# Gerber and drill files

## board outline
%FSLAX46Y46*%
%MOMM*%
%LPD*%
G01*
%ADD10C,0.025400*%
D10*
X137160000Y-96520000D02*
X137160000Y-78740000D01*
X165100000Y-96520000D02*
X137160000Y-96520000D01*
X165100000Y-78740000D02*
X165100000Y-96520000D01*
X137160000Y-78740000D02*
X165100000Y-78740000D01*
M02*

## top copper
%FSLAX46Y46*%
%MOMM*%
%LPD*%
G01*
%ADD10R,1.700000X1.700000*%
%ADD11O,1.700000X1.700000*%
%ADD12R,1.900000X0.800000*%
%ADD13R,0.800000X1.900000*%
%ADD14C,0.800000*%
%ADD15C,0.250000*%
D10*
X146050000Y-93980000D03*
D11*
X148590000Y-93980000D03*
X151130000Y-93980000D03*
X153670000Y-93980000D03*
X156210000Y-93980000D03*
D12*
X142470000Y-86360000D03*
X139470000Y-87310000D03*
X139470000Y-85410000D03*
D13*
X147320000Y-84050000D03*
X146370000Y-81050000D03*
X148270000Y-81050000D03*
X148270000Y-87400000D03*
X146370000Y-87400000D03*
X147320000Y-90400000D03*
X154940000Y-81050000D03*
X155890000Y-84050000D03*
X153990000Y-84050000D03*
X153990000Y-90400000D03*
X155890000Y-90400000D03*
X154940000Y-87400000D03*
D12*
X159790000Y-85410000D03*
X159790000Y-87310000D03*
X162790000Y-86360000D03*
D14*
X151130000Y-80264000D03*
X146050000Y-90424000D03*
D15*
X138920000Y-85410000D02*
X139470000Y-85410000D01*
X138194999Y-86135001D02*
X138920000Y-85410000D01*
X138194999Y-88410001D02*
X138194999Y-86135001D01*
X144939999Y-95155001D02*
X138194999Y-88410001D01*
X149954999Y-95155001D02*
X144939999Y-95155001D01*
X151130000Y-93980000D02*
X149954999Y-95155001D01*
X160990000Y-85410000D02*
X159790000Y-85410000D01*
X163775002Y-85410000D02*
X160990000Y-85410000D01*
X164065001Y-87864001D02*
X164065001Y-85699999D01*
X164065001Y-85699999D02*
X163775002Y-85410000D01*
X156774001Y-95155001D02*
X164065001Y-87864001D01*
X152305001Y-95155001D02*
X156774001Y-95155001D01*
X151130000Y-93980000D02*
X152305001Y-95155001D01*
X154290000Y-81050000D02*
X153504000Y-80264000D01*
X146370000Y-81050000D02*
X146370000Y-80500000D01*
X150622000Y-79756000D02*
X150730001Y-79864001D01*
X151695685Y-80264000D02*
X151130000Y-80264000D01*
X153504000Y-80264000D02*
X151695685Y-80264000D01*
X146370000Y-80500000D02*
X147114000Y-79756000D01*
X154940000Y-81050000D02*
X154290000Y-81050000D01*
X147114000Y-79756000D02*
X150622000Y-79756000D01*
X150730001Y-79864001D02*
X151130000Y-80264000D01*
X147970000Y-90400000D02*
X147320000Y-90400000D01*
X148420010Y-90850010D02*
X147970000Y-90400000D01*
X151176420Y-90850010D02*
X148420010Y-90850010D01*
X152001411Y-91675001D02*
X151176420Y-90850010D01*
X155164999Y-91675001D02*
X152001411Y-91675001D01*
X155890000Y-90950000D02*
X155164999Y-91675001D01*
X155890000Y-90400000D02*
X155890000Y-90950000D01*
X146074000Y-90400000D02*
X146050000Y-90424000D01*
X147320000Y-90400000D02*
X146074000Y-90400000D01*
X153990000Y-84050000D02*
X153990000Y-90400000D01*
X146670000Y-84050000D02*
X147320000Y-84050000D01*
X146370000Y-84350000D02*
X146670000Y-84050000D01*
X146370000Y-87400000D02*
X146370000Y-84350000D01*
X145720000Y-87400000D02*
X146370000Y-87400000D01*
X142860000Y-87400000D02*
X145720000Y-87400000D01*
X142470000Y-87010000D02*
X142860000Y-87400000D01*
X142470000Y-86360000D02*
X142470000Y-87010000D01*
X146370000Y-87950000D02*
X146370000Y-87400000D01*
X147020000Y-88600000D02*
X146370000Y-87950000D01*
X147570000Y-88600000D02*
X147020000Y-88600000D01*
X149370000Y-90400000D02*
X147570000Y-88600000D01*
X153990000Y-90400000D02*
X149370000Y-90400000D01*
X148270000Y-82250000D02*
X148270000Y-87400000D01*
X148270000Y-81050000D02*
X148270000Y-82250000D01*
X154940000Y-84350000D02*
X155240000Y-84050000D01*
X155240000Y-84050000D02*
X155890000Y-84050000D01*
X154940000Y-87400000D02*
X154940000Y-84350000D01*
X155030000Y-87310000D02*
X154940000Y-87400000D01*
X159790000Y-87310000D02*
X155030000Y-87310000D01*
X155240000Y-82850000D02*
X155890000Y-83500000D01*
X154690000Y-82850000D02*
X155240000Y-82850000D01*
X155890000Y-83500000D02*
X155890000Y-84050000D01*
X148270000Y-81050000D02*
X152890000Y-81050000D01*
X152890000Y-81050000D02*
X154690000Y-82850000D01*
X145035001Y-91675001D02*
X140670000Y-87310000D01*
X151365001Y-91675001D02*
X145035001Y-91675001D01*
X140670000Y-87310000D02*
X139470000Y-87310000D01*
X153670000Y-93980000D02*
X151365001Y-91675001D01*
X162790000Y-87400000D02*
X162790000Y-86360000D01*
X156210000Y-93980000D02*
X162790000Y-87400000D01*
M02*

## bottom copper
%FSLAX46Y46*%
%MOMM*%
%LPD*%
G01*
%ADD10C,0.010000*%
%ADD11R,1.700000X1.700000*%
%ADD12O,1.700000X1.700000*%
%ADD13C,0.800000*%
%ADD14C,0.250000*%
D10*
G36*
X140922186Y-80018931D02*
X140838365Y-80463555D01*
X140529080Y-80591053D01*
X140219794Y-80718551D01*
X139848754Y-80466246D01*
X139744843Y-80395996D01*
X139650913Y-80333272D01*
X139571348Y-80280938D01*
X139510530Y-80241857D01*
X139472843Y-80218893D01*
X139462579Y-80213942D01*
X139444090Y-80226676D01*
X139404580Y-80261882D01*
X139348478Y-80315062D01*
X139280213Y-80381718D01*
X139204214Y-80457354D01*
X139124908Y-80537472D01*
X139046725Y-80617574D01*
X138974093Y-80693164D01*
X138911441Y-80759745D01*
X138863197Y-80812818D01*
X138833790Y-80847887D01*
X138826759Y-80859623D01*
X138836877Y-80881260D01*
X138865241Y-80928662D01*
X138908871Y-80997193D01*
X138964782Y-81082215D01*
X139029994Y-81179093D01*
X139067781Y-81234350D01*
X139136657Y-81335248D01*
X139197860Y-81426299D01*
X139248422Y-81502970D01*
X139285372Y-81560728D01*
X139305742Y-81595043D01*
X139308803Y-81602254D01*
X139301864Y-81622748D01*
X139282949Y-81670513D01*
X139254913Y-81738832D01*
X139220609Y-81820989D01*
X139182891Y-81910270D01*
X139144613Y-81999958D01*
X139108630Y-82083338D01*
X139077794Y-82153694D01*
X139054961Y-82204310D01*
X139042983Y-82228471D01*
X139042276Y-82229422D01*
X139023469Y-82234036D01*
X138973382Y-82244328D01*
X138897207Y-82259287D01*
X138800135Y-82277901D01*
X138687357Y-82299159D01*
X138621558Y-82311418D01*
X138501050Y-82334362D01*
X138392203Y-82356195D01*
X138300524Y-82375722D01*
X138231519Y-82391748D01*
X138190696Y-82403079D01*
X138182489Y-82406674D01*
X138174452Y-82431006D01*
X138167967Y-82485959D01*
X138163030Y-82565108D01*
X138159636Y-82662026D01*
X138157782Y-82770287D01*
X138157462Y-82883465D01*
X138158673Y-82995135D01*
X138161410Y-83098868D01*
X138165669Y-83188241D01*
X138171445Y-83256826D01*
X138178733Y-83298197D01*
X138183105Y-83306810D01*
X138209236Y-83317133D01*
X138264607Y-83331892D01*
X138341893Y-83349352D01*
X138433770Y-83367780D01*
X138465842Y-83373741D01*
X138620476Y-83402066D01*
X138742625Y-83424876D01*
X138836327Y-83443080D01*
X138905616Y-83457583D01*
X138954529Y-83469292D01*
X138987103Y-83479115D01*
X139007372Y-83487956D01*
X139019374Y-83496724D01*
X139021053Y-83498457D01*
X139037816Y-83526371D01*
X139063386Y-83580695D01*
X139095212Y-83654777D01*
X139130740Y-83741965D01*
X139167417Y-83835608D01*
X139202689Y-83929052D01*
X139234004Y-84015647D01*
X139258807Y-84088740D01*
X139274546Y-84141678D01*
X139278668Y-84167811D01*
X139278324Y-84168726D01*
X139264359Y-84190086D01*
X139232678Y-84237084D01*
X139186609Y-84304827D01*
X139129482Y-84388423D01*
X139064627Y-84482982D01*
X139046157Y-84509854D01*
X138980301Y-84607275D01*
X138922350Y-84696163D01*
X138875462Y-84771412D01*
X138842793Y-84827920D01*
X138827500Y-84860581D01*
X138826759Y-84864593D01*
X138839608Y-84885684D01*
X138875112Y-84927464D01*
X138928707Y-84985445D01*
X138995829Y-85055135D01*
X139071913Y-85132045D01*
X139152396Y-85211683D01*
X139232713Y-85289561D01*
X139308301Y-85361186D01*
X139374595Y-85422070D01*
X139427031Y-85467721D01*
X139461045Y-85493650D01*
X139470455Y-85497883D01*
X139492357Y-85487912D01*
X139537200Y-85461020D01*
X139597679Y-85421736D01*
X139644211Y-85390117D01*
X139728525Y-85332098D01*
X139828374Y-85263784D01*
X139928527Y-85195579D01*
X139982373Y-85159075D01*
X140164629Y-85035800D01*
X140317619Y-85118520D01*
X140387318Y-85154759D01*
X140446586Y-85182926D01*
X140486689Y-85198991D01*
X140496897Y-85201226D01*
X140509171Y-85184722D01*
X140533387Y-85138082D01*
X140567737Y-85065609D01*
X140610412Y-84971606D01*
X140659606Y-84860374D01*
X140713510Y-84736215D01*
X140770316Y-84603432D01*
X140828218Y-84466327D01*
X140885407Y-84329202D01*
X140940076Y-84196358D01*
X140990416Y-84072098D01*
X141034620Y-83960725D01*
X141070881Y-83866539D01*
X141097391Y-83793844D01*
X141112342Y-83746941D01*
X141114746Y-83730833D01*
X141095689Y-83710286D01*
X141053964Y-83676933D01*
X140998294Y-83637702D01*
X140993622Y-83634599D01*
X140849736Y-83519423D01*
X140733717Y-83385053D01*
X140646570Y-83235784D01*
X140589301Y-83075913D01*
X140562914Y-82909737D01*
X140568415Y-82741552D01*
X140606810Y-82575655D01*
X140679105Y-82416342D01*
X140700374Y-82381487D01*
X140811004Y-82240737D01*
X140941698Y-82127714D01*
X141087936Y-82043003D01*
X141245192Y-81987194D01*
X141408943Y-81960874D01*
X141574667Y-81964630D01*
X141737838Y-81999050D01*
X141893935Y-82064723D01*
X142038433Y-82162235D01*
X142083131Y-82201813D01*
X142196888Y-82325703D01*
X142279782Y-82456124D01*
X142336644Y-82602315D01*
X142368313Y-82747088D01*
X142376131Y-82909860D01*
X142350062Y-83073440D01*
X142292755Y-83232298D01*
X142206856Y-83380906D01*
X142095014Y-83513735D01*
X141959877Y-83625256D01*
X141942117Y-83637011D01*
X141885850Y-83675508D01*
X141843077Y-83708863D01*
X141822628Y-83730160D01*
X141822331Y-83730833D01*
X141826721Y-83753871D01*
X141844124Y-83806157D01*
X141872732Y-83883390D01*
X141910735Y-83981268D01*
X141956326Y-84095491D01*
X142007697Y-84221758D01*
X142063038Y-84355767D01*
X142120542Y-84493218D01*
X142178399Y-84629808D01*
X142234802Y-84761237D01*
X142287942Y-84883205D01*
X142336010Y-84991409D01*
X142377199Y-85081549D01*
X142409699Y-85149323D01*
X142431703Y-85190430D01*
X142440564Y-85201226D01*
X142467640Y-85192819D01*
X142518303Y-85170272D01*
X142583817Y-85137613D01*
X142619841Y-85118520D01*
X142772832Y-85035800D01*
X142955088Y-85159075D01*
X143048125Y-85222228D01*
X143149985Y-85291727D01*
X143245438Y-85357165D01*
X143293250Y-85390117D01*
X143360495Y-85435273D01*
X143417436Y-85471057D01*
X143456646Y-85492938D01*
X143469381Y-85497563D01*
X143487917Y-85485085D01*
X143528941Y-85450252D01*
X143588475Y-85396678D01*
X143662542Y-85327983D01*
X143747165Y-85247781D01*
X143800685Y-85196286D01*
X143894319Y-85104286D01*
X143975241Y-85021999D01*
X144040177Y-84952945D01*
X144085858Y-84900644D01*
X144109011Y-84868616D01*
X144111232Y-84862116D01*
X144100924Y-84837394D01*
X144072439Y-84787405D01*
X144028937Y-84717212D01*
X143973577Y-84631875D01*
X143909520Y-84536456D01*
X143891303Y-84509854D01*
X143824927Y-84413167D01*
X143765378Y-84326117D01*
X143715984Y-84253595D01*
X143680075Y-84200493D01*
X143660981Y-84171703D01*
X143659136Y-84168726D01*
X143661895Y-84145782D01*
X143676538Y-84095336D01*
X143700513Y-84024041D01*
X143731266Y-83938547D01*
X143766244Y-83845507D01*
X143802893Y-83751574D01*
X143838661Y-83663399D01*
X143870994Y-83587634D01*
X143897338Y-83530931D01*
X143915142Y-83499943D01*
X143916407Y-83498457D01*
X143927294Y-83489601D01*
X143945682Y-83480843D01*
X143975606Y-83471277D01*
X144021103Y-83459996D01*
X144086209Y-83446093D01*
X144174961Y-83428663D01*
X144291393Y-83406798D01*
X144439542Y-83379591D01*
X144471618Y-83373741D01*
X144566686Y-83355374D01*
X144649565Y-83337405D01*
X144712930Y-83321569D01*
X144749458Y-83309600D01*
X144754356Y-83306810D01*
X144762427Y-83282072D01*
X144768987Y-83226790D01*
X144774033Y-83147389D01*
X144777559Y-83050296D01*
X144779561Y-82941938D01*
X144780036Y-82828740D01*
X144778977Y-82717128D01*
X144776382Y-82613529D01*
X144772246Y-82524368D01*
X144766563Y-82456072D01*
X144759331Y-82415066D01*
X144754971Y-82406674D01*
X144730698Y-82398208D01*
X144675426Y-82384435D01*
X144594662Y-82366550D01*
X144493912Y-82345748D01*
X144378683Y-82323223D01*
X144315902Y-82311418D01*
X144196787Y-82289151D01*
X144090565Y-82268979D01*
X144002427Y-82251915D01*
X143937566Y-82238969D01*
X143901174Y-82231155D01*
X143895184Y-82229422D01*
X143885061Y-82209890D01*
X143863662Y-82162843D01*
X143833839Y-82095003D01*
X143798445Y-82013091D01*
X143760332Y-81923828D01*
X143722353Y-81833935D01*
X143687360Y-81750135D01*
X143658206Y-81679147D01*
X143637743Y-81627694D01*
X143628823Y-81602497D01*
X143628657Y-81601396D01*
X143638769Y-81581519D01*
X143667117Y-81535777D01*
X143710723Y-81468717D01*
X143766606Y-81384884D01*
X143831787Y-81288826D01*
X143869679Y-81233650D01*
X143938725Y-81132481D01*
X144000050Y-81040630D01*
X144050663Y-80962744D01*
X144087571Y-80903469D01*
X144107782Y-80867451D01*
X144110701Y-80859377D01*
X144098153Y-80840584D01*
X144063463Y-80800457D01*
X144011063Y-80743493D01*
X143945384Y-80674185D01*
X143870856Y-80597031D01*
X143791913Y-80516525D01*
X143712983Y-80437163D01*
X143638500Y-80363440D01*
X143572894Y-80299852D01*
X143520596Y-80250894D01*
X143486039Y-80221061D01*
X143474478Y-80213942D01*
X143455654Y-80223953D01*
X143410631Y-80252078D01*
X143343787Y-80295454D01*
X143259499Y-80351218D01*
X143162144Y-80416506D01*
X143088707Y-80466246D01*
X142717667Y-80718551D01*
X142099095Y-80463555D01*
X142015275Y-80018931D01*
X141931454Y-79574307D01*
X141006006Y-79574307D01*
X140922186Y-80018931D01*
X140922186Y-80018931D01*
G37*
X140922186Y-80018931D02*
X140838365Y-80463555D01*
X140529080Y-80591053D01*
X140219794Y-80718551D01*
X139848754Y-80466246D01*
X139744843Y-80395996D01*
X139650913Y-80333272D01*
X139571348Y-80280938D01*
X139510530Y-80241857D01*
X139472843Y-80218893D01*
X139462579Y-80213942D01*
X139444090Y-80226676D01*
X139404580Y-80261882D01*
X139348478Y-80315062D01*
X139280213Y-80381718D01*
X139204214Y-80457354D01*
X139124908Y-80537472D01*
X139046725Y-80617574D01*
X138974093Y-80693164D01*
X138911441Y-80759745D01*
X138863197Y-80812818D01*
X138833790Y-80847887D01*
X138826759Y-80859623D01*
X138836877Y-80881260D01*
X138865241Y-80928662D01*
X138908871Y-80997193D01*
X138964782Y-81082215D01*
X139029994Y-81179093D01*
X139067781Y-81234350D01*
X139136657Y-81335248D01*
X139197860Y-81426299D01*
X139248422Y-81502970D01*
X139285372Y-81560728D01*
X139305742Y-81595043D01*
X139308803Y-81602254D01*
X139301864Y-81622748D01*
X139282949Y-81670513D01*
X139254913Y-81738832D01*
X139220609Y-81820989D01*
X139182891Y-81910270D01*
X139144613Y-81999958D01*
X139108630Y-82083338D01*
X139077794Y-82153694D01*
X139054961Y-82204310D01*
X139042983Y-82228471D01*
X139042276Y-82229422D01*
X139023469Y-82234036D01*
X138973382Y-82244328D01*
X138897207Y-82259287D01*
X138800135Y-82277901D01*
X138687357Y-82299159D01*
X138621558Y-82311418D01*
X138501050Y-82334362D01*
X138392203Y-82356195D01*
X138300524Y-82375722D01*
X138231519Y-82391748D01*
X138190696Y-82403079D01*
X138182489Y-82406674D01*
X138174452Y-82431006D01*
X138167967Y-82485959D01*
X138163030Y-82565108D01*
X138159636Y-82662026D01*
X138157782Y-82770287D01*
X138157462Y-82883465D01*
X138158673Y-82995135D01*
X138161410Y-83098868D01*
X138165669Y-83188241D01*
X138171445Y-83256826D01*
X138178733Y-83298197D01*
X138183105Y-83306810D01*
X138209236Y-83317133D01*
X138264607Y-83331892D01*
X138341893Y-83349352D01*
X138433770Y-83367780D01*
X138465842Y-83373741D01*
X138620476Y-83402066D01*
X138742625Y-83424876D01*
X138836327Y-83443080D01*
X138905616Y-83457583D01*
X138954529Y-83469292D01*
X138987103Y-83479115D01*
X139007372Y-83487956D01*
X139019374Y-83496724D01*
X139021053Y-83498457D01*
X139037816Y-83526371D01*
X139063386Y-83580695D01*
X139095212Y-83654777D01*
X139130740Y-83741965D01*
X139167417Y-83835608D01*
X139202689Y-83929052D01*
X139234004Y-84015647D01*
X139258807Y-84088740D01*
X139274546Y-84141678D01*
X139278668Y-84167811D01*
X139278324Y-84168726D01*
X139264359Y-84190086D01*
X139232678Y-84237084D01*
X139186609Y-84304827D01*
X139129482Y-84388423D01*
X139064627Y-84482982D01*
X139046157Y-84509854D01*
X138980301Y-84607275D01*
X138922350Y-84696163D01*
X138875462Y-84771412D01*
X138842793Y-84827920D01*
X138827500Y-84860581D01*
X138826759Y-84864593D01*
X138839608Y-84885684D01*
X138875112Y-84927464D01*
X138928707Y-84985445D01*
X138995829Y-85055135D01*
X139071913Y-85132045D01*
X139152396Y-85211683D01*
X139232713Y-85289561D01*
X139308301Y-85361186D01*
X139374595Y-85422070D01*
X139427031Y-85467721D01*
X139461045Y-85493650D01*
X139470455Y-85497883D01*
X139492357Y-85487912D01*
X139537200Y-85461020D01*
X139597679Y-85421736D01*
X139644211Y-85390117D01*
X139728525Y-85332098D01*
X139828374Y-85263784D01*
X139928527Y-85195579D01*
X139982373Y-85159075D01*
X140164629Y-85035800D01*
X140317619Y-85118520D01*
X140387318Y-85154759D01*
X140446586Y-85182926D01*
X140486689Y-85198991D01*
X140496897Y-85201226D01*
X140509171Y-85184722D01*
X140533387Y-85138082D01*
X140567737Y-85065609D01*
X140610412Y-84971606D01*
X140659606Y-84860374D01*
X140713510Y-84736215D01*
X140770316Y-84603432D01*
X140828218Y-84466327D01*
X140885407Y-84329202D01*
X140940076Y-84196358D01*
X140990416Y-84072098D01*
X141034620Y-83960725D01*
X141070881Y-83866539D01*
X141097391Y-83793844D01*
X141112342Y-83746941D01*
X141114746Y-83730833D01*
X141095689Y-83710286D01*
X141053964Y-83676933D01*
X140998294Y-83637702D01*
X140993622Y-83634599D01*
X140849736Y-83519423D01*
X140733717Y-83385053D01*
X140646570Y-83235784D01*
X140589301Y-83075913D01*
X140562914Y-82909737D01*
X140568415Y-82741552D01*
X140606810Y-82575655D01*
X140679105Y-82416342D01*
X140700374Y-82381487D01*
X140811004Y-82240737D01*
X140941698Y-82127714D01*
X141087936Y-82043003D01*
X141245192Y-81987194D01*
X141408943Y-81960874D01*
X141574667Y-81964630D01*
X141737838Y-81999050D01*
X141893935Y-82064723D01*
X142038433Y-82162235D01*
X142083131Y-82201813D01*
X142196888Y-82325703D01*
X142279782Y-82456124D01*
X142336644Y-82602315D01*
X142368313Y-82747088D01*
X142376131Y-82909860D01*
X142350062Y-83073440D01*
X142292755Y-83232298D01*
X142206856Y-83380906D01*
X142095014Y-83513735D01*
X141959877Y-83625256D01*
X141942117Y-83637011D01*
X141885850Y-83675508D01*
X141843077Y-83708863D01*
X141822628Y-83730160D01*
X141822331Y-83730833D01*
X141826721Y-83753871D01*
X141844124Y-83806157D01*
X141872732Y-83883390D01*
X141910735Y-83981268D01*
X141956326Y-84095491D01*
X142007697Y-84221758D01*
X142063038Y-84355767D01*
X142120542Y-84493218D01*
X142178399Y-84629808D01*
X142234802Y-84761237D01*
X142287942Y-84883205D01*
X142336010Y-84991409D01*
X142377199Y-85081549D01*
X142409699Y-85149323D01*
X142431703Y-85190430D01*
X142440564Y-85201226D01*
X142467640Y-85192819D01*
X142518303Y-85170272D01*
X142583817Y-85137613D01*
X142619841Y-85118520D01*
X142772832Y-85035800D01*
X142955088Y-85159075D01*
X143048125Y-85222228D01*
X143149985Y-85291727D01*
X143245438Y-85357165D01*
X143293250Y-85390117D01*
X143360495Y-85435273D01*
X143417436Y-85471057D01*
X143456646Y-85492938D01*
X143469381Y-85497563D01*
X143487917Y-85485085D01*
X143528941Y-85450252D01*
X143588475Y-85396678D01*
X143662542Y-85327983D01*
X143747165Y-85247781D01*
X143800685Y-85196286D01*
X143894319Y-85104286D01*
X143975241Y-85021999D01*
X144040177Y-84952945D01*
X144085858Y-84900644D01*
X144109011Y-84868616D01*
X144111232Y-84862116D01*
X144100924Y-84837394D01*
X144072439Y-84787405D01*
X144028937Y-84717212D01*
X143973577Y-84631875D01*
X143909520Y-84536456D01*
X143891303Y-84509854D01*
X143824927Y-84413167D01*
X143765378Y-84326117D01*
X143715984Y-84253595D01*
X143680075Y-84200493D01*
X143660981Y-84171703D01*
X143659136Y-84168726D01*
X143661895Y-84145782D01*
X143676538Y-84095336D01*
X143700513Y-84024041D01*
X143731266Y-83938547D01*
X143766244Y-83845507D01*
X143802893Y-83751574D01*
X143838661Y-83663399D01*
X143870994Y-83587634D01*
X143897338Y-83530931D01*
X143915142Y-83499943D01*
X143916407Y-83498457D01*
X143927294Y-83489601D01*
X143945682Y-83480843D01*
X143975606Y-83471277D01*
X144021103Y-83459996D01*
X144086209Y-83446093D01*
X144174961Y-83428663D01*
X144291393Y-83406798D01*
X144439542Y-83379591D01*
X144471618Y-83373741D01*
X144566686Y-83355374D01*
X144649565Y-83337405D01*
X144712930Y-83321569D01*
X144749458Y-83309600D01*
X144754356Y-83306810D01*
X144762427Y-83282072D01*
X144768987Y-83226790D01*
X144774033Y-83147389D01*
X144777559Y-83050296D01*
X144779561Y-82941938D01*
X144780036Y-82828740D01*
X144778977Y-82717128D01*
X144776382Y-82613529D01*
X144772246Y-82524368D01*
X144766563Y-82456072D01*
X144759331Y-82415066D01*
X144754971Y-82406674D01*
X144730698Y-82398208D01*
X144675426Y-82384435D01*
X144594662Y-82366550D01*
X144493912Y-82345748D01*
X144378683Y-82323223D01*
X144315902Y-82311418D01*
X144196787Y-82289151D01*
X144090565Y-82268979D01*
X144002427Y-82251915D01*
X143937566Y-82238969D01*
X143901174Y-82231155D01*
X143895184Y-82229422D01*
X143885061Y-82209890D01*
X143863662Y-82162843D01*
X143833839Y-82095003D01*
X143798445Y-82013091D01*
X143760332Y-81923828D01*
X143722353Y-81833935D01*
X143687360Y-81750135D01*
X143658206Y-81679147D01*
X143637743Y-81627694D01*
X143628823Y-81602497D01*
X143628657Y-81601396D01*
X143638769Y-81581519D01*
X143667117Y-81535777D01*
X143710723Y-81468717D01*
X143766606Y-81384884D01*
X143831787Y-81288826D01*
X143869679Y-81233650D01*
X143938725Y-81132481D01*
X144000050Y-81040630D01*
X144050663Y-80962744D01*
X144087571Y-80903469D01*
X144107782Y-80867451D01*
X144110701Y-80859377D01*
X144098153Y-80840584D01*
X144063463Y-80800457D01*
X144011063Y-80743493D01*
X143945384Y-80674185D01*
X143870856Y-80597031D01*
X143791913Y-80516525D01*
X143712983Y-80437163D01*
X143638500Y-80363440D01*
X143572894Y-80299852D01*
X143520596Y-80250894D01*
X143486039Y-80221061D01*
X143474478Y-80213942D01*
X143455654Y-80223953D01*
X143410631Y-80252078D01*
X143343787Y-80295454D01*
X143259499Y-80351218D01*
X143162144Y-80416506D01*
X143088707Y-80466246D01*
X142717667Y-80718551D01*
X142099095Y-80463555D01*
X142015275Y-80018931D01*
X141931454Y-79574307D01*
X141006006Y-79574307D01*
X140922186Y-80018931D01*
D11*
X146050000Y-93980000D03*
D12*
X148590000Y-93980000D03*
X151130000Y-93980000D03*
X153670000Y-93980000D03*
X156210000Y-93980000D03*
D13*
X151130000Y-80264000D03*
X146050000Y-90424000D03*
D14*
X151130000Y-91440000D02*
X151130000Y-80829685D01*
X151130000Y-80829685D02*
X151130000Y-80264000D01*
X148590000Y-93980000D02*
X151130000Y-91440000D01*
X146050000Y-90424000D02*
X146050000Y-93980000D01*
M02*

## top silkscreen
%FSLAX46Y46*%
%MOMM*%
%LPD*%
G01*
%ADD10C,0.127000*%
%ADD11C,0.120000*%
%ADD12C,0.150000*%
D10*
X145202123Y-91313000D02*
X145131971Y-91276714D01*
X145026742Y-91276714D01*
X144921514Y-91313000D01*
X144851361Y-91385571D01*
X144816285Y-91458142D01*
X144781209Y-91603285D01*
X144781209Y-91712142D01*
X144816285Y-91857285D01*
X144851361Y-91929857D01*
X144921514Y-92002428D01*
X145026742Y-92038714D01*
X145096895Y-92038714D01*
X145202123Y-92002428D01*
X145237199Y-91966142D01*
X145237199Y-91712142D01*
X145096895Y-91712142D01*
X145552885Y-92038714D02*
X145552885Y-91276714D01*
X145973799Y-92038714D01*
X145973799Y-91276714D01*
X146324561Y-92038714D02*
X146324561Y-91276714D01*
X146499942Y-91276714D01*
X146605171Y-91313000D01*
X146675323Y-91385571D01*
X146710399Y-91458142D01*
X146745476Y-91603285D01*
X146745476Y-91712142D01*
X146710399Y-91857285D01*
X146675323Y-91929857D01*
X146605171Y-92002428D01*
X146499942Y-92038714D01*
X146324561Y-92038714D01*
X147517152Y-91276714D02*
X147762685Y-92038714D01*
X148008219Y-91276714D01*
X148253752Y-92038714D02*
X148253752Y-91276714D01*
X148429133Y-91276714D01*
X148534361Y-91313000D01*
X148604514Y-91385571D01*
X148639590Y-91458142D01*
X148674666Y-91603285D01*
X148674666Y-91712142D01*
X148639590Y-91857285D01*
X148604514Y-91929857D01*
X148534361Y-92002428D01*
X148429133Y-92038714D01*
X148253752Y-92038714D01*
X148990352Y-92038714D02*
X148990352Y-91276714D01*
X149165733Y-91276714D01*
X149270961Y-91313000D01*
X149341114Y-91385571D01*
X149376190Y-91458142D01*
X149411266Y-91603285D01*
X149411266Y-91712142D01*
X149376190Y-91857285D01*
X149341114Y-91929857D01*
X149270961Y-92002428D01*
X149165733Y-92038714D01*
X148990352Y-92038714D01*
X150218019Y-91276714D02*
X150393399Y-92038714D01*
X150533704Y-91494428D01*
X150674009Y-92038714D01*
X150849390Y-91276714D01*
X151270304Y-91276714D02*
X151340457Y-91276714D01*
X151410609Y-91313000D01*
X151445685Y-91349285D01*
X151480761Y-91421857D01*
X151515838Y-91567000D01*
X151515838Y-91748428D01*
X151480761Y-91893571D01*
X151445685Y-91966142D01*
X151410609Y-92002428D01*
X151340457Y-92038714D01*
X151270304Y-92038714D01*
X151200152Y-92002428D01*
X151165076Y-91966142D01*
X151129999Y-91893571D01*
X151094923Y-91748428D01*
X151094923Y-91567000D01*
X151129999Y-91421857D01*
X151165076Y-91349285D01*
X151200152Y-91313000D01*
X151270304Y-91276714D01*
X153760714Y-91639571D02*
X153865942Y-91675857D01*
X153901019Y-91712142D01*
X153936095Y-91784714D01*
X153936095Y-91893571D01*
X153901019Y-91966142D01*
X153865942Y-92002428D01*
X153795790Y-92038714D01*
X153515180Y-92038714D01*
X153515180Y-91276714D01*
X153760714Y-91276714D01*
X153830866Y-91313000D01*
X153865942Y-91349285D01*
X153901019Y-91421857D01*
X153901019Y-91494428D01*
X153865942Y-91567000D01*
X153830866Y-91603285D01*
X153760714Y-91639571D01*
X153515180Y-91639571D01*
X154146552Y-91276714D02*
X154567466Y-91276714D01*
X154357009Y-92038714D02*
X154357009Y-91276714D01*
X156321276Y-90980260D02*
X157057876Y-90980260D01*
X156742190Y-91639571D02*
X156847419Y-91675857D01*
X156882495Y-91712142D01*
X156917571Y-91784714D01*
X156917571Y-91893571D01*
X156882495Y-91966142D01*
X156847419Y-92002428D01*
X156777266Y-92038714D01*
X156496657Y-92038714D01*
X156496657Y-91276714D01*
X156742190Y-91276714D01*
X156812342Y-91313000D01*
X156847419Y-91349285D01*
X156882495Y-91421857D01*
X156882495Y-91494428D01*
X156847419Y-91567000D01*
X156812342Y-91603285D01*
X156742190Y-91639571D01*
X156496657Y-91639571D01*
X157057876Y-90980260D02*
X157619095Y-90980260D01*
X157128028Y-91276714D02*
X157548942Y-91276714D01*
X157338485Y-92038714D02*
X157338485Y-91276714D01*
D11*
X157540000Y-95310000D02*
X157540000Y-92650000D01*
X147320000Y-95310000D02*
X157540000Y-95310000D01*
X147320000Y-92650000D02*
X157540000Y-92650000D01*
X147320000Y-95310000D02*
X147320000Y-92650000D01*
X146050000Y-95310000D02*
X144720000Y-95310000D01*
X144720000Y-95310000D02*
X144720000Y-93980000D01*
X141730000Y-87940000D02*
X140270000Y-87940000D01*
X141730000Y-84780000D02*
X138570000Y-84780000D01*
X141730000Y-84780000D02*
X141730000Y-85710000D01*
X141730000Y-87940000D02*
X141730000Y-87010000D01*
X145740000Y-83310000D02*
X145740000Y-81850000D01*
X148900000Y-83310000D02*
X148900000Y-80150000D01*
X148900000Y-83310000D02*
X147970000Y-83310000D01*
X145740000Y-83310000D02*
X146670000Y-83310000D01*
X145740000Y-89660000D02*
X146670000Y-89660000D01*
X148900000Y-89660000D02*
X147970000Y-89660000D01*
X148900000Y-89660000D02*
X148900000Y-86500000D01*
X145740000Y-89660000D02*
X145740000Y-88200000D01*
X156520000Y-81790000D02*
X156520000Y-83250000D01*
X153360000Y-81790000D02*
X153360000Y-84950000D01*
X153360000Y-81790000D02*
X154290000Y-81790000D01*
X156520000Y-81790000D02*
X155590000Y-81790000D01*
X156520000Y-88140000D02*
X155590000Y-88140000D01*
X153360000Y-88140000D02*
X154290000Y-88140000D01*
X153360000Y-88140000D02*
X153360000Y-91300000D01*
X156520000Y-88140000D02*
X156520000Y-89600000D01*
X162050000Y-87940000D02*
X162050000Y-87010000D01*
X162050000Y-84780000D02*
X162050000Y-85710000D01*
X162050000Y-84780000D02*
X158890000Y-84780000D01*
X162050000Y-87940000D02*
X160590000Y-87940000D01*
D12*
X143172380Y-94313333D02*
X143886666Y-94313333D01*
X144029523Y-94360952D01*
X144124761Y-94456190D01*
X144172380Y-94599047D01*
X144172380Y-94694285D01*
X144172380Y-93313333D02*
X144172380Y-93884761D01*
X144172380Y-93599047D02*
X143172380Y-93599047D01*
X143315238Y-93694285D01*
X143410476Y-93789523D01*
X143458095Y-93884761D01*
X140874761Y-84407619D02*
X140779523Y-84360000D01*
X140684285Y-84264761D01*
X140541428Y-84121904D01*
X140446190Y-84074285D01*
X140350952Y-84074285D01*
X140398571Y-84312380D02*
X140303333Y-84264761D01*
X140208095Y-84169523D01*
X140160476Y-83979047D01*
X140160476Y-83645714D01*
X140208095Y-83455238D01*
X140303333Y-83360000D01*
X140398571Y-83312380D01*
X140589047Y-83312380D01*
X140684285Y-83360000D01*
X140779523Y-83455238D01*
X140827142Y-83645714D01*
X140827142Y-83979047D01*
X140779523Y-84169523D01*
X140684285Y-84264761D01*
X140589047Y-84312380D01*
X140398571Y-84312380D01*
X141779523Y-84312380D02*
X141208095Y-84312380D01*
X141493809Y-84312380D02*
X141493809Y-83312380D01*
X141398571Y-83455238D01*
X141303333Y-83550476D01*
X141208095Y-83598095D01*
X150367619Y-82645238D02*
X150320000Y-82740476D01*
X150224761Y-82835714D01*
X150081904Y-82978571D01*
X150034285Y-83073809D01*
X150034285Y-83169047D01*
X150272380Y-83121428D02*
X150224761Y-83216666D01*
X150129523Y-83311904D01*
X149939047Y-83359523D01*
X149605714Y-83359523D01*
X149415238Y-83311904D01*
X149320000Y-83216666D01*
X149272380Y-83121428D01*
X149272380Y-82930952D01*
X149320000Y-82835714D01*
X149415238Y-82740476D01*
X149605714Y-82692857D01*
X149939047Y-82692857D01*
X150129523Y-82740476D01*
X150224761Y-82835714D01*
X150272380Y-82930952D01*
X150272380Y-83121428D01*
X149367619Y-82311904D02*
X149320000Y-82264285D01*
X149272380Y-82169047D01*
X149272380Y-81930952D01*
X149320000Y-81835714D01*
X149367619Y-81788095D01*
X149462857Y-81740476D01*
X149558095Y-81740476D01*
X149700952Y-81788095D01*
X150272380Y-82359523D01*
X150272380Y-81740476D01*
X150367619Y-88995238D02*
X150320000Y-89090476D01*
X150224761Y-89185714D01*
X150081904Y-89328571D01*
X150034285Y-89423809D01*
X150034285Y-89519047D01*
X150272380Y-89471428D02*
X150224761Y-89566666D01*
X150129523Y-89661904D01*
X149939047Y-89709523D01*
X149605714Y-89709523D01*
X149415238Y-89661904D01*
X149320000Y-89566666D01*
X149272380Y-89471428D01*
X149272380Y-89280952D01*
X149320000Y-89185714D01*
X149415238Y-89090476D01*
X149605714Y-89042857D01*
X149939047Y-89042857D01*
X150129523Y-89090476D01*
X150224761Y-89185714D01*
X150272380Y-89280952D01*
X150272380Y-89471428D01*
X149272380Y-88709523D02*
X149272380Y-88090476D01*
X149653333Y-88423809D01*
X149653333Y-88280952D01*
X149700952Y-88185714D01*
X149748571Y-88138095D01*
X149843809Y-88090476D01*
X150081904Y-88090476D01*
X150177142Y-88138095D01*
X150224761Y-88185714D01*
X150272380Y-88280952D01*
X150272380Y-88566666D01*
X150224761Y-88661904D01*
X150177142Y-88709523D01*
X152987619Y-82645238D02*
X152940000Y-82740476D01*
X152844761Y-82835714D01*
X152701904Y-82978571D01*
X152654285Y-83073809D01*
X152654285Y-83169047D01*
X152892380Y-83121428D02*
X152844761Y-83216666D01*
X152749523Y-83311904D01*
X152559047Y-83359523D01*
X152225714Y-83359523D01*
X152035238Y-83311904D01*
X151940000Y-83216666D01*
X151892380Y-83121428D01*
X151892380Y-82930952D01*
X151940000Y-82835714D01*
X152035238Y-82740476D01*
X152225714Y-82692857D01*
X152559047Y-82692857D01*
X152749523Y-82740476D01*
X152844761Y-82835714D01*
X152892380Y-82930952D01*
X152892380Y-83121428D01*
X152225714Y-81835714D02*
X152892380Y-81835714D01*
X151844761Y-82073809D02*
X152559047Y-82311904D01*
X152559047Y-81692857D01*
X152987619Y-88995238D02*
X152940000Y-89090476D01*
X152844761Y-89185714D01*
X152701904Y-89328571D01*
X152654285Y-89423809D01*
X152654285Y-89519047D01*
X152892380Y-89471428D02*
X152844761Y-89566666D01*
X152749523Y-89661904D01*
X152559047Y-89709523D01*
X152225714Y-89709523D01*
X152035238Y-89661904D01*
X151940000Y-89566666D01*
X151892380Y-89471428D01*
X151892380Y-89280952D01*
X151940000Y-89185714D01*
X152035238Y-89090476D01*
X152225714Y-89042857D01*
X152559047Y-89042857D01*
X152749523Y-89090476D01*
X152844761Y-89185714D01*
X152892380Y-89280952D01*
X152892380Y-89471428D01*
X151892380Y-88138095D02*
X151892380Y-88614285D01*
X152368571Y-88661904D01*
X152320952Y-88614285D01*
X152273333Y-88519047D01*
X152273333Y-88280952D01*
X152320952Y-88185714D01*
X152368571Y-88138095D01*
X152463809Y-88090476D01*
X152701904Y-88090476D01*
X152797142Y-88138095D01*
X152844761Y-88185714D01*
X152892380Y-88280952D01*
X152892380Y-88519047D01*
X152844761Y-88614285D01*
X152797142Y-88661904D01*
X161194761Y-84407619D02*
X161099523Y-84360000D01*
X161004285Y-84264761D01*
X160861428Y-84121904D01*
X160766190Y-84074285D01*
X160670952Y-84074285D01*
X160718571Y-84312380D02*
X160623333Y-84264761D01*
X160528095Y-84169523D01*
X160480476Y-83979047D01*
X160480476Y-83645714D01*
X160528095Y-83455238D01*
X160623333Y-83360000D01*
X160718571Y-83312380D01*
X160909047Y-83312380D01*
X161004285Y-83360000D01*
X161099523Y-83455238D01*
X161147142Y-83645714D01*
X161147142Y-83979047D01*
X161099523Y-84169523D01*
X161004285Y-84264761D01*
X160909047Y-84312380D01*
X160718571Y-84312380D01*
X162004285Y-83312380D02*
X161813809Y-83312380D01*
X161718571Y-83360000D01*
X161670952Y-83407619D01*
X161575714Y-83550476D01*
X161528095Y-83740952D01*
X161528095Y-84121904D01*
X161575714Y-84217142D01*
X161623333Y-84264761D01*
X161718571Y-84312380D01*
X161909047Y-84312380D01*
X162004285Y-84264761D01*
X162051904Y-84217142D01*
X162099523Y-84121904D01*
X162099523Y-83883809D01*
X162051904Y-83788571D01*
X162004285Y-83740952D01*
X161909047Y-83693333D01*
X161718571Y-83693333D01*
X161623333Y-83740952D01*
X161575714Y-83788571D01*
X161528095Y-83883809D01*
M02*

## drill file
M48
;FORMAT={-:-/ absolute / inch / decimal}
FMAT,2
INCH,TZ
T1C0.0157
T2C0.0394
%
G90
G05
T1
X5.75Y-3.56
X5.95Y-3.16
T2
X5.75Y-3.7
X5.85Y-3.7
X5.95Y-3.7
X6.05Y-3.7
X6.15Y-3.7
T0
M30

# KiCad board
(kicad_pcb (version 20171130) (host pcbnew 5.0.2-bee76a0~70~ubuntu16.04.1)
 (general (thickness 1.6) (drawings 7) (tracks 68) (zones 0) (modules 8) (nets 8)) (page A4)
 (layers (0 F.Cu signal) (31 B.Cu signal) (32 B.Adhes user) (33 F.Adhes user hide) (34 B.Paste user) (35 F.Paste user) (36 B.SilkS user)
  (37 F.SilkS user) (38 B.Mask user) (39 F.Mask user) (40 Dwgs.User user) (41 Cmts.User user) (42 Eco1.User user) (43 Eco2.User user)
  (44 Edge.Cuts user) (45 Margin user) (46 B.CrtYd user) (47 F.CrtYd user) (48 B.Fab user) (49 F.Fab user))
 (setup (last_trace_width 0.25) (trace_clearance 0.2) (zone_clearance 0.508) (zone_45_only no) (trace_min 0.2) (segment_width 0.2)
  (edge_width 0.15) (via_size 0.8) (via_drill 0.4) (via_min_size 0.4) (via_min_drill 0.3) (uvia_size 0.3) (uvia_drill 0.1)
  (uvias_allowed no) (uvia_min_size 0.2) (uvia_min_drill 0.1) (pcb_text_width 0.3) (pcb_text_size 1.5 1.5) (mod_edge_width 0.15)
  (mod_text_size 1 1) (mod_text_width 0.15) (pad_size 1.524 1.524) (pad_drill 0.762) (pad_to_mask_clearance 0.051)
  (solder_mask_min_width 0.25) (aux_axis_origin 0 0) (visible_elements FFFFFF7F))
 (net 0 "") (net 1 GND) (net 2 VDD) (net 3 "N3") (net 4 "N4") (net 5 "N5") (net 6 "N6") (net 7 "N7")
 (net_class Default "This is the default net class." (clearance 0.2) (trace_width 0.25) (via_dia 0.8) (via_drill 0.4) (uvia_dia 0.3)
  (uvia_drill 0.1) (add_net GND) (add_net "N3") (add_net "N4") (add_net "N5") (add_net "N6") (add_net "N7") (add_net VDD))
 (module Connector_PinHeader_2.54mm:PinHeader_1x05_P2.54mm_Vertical (layer F.Cu) (at 146.05 93.98 90)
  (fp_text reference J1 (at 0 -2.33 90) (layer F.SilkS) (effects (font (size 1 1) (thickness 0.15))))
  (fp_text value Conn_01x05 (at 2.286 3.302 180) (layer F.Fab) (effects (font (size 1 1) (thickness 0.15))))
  (fp_line (start -1.33 11.49) (end 1.33 11.49) (layer F.SilkS) (width 0.12))
  (fp_line (start -1.33 1.27) (end -1.33 11.49) (layer F.SilkS) (width 0.12))
  (fp_line (start 1.33 1.27) (end 1.33 11.49) (layer F.SilkS) (width 0.12))
  (fp_line (start -1.33 1.27) (end 1.33 1.27) (layer F.SilkS) (width 0.12))
  (fp_line (start -1.33 0) (end -1.33 -1.33) (layer F.SilkS) (width 0.12))
  (fp_line (start -1.33 -1.33) (end 0 -1.33) (layer F.SilkS) (width 0.12))
  (pad 1 thru_hole rect (at 0 0 90) (size 1.7 1.7) (drill 1) (layers *.Cu *.Mask) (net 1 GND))
  (pad 2 thru_hole oval (at 0 2.54 90) (size 1.7 1.7) (drill 1) (layers *.Cu *.Mask) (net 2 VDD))
  (pad 3 thru_hole oval (at 0 5.08 90) (size 1.7 1.7) (drill 1) (layers *.Cu *.Mask) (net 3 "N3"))
  (pad 4 thru_hole oval (at 0 7.62 90) (size 1.7 1.7) (drill 1) (layers *.Cu *.Mask) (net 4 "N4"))
  (pad 5 thru_hole oval (at 0 10.16 90) (size 1.7 1.7) (drill 1) (layers *.Cu *.Mask) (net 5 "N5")))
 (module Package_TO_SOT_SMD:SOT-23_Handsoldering (layer F.Cu) (at 140.97 86.36)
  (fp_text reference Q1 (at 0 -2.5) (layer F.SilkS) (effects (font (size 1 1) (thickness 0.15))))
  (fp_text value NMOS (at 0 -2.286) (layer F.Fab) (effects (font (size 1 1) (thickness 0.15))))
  (fp_line (start 0.76 1.58) (end -0.7 1.58) (layer F.SilkS) (width 0.12))
  (fp_line (start 0.76 -1.58) (end -2.4 -1.58) (layer F.SilkS) (width 0.12))
  (fp_line (start 0.76 -1.58) (end 0.76 -0.65) (layer F.SilkS) (width 0.12))
  (fp_line (start 0.76 1.58) (end 0.76 0.65) (layer F.SilkS) (width 0.12))
  (pad 3 smd rect (at 1.5 0) (size 1.9 0.8) (layers F.Cu F.Paste F.Mask) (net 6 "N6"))
  (pad 2 smd rect (at -1.5 0.95) (size 1.9 0.8) (layers F.Cu F.Paste F.Mask) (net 4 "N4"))
  (pad 1 smd rect (at -1.5 -0.95) (size 1.9 0.8) (layers F.Cu F.Paste F.Mask) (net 3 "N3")))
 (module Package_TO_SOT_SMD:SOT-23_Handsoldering (layer F.Cu) (at 147.32 82.55 270)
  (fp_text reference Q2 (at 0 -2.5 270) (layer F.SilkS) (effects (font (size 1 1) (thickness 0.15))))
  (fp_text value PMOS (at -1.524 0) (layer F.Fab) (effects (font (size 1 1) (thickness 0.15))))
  (fp_line (start 0.76 1.58) (end -0.7 1.58) (layer F.SilkS) (width 0.12))
  (fp_line (start 0.76 -1.58) (end -2.4 -1.58) (layer F.SilkS) (width 0.12))
  (fp_line (start 0.76 -1.58) (end 0.76 -0.65) (layer F.SilkS) (width 0.12))
  (fp_line (start 0.76 1.58) (end 0.76 0.65) (layer F.SilkS) (width 0.12))
  (pad 3 smd rect (at 1.5 0 270) (size 1.9 0.8) (layers F.Cu F.Paste F.Mask) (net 6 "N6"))
  (pad 2 smd rect (at -1.5 0.95 270) (size 1.9 0.8) (layers F.Cu F.Paste F.Mask) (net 2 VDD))
  (pad 1 smd rect (at -1.5 -0.95 270) (size 1.9 0.8) (layers F.Cu F.Paste F.Mask) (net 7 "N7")))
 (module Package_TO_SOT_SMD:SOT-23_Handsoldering (layer F.Cu) (at 147.32 88.9 270)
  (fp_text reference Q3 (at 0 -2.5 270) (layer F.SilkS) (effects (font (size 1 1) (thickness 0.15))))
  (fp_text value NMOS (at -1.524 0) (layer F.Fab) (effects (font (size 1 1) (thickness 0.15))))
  (fp_line (start 0.76 1.58) (end 0.76 0.65) (layer F.SilkS) (width 0.12))
  (fp_line (start 0.76 -1.58) (end 0.76 -0.65) (layer F.SilkS) (width 0.12))
  (fp_line (start 0.76 -1.58) (end -2.4 -1.58) (layer F.SilkS) (width 0.12))
  (fp_line (start 0.76 1.58) (end -0.7 1.58) (layer F.SilkS) (width 0.12))
  (pad 1 smd rect (at -1.5 -0.95 270) (size 1.9 0.8) (layers F.Cu F.Paste F.Mask) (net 7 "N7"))
  (pad 2 smd rect (at -1.5 0.95 270) (size 1.9 0.8) (layers F.Cu F.Paste F.Mask) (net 6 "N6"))
  (pad 3 smd rect (at 1.5 0 270) (size 1.9 0.8) (layers F.Cu F.Paste F.Mask) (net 1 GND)))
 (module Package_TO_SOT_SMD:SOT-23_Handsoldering (layer F.Cu) (at 154.94 82.55 90)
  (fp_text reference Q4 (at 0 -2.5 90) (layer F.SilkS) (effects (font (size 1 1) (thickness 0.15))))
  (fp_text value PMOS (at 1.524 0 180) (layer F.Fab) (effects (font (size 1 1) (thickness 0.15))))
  (fp_line (start 0.76 1.58) (end -0.7 1.58) (layer F.SilkS) (width 0.12))
  (fp_line (start 0.76 -1.58) (end -2.4 -1.58) (layer F.SilkS) (width 0.12))
  (fp_line (start 0.76 -1.58) (end 0.76 -0.65) (layer F.SilkS) (width 0.12))
  (fp_line (start 0.76 1.58) (end 0.76 0.65) (layer F.SilkS) (width 0.12))
  (pad 3 smd rect (at 1.5 0 90) (size 1.9 0.8) (layers F.Cu F.Paste F.Mask) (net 2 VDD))
  (pad 2 smd rect (at -1.5 0.95 90) (size 1.9 0.8) (layers F.Cu F.Paste F.Mask) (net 7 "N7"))
  (pad 1 smd rect (at -1.5 -0.95 90) (size 1.9 0.8) (layers F.Cu F.Paste F.Mask) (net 6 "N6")))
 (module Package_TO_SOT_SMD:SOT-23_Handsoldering (layer F.Cu) (at 154.94 88.9 90)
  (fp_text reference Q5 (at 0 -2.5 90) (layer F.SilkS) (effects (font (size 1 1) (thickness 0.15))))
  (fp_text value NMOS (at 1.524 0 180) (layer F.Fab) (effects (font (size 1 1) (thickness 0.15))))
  (fp_line (start 0.76 1.58) (end 0.76 0.65) (layer F.SilkS) (width 0.12))
  (fp_line (start 0.76 -1.58) (end 0.76 -0.65) (layer F.SilkS) (width 0.12))
  (fp_line (start 0.76 -1.58) (end -2.4 -1.58) (layer F.SilkS) (width 0.12))
  (fp_line (start 0.76 1.58) (end -0.7 1.58) (layer F.SilkS) (width 0.12))
  (pad 1 smd rect (at -1.5 -0.95 90) (size 1.9 0.8) (layers F.Cu F.Paste F.Mask) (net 6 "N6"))
  (pad 2 smd rect (at -1.5 0.95 90) (size 1.9 0.8) (layers F.Cu F.Paste F.Mask) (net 1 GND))
  (pad 3 smd rect (at 1.5 0 90) (size 1.9 0.8) (layers F.Cu F.Paste F.Mask) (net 7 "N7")))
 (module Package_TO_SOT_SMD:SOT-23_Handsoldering (layer F.Cu) (at 161.29 86.36)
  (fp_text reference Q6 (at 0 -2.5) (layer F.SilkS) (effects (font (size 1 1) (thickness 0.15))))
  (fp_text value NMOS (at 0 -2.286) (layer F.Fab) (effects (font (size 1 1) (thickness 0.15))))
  (fp_line (start 0.76 1.58) (end 0.76 0.65) (layer F.SilkS) (width 0.12))
  (fp_line (start 0.76 -1.58) (end 0.76 -0.65) (layer F.SilkS) (width 0.12))
  (fp_line (start 0.76 -1.58) (end -2.4 -1.58) (layer F.SilkS) (width 0.12))
  (fp_line (start 0.76 1.58) (end -0.7 1.58) (layer F.SilkS) (width 0.12))
  (pad 1 smd rect (at -1.5 -0.95) (size 1.9 0.8) (layers F.Cu F.Paste F.Mask) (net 3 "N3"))
  (pad 2 smd rect (at -1.5 0.95) (size 1.9 0.8) (layers F.Cu F.Paste F.Mask) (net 7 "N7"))
  (pad 3 smd rect (at 1.5 0) (size 1.9 0.8) (layers F.Cu F.Paste F.Mask) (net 5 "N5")))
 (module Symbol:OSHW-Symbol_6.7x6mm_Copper (layer B.Cu) (at 141.478 82.55 180)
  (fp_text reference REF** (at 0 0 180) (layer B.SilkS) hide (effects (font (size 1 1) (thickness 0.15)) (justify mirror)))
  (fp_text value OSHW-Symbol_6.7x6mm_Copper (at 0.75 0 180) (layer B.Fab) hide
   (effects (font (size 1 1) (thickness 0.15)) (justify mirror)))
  (fp_poly
   (pts (xy 0.555814 2.531069) (xy 0.639635 2.086445) (xy 0.94892 1.958947) (xy 1.258206 1.831449) (xy 1.629246 2.083754)
    (xy 1.733157 2.154004) (xy 1.827087 2.216728) (xy 1.906652 2.269062) (xy 1.96747 2.308143) (xy 2.005157 2.331107) (xy 2.015421 2.336058)
    (xy 2.03391 2.323324) (xy 2.07342 2.288118) (xy 2.129522 2.234938) (xy 2.197787 2.168282) (xy 2.273786 2.092646) (xy 2.353092 2.012528)
    (xy 2.431275 1.932426) (xy 2.503907 1.856836) (xy 2.566559 1.790255) (xy 2.614803 1.737182) (xy 2.64421 1.702113) (xy 2.651241 1.690377)
    (xy 2.641123 1.66874) (xy 2.612759 1.621338) (xy 2.569129 1.552807) (xy 2.513218 1.467785) (xy 2.448006 1.370907) (xy 2.410219 1.31565)
    (xy 2.341343 1.214752) (xy 2.28014 1.123701) (xy 2.229578 1.04703) (xy 2.192628 0.989272) (xy 2.172258 0.954957) (xy 2.169197 0.947746)
    (xy 2.176136 0.927252) (xy 2.195051 0.879487) (xy 2.223087 0.811168) (xy 2.257391 0.729011) (xy 2.295109 0.63973) (xy 2.333387 0.550042)
    (xy 2.36937 0.466662) (xy 2.400206 0.396306) (xy 2.423039 0.34569) (xy 2.435017 0.321529) (xy 2.435724 0.320578) (xy 2.454531 0.315964)
    (xy 2.504618 0.305672) (xy 2.580793 0.290713) (xy 2.677865 0.272099) (xy 2.790643 0.250841) (xy 2.856442 0.238582) (xy 2.97695 0.215638)
    (xy 3.085797 0.193805) (xy 3.177476 0.174278) (xy 3.246481 0.158252) (xy 3.287304 0.146921) (xy 3.295511 0.143326)
    (xy 3.303548 0.118994) (xy 3.310033 0.064041) (xy 3.31497 -0.015108) (xy 3.318364 -0.112026) (xy 3.320218 -0.220287)
    (xy 3.320538 -0.333465) (xy 3.319327 -0.445135) (xy 3.31659 -0.548868) (xy 3.312331 -0.638241) (xy 3.306555 -0.706826)
    (xy 3.299267 -0.748197) (xy 3.294895 -0.75681) (xy 3.268764 -0.767133) (xy 3.213393 -0.781892) (xy 3.136107 -0.799352)
    (xy 3.04423 -0.81778) (xy 3.012158 -0.823741) (xy 2.857524 -0.852066) (xy 2.735375 -0.874876) (xy 2.641673 -0.89308)
    (xy 2.572384 -0.907583) (xy 2.523471 -0.919292) (xy 2.490897 -0.929115) (xy 2.470628 -0.937956) (xy 2.458626 -0.946724)
    (xy 2.456947 -0.948457) (xy 2.440184 -0.976371) (xy 2.414614 -1.030695) (xy 2.382788 -1.104777) (xy 2.34726 -1.191965)
    (xy 2.310583 -1.285608) (xy 2.275311 -1.379052) (xy 2.243996 -1.465647) (xy 2.219193 -1.53874) (xy 2.203454 -1.591678)
    (xy 2.199332 -1.617811) (xy 2.199676 -1.618726) (xy 2.213641 -1.640086) (xy 2.245322 -1.687084) (xy 2.291391 -1.754827)
    (xy 2.348518 -1.838423) (xy 2.413373 -1.932982) (xy 2.431843 -1.959854) (xy 2.497699 -2.057275) (xy 2.55565 -2.146163)
    (xy 2.602538 -2.221412) (xy 2.635207 -2.27792) (xy 2.6505 -2.310581) (xy 2.651241 -2.314593) (xy 2.638392 -2.335684)
    (xy 2.602888 -2.377464) (xy 2.549293 -2.435445) (xy 2.482171 -2.505135) (xy 2.406087 -2.582045) (xy 2.325604 -2.661683)
    (xy 2.245287 -2.739561) (xy 2.169699 -2.811186) (xy 2.103405 -2.87207) (xy 2.050969 -2.917721) (xy 2.016955 -2.94365)
    (xy 2.007545 -2.947883) (xy 1.985643 -2.937912) (xy 1.9408 -2.91102) (xy 1.880321 -2.871736) (xy 1.833789 -2.840117)
    (xy 1.749475 -2.782098) (xy 1.649626 -2.713784) (xy 1.549473 -2.645579) (xy 1.495627 -2.609075) (xy 1.313371 -2.4858)
    (xy 1.160381 -2.56852) (xy 1.090682 -2.604759) (xy 1.031414 -2.632926) (xy 0.991311 -2.648991) (xy 0.981103 -2.651226)
    (xy 0.968829 -2.634722) (xy 0.944613 -2.588082) (xy 0.910263 -2.515609) (xy 0.867588 -2.421606) (xy 0.818394 -2.310374)
    (xy 0.76449 -2.186215) (xy 0.707684 -2.053432) (xy 0.649782 -1.916327) (xy 0.592593 -1.779202) (xy 0.537924 -1.646358)
    (xy 0.487584 -1.522098) (xy 0.44338 -1.410725) (xy 0.407119 -1.316539) (xy 0.380609 -1.243844) (xy 0.365658 -1.196941)
    (xy 0.363254 -1.180833) (xy 0.382311 -1.160286) (xy 0.424036 -1.126933) (xy 0.479706 -1.087702) (xy 0.484378 -1.084599)
    (xy 0.628264 -0.969423) (xy 0.744283 -0.835053) (xy 0.83143 -0.685784) (xy 0.888699 -0.525913) (xy 0.915086 -0.359737)
    (xy 0.909585 -0.191552) (xy 0.87119 -0.025655) (xy 0.798895 0.133658) (xy 0.777626 0.168513) (xy 0.666996 0.309263)
    (xy 0.536302 0.422286) (xy 0.390064 0.506997) (xy 0.232808 0.562806) (xy 0.069057 0.589126) (xy -0.096667 0.58537)
    (xy -0.259838 0.55095) (xy -0.415935 0.485277) (xy -0.560433 0.387765) (xy -0.605131 0.348187) (xy -0.718888 0.224297)
    (xy -0.801782 0.093876) (xy -0.858644 -0.052315) (xy -0.890313 -0.197088) (xy -0.898131 -0.35986) (xy -0.872062 -0.52344)
    (xy -0.814755 -0.682298) (xy -0.728856 -0.830906) (xy -0.617014 -0.963735) (xy -0.481877 -1.075256) (xy -0.464117 -1.087011)
    (xy -0.40785 -1.125508) (xy -0.365077 -1.158863) (xy -0.344628 -1.18016) (xy -0.344331 -1.180833) (xy -0.348721 -1.203871)
    (xy -0.366124 -1.256157) (xy -0.394732 -1.33339) (xy -0.432735 -1.431268) (xy -0.478326 -1.545491) (xy -0.529697 -1.671758)
    (xy -0.585038 -1.805767) (xy -0.642542 -1.943218) (xy -0.700399 -2.079808) (xy -0.756802 -2.211237) (xy -0.809942 -2.333205)
    (xy -0.85801 -2.441409) (xy -0.899199 -2.531549) (xy -0.931699 -2.599323) (xy -0.953703 -2.64043) (xy -0.962564 -2.651226)
    (xy -0.98964 -2.642819) (xy -1.040303 -2.620272) (xy -1.105817 -2.587613) (xy -1.141841 -2.56852) (xy -1.294832 -2.4858)
    (xy -1.477088 -2.609075) (xy -1.570125 -2.672228) (xy -1.671985 -2.741727) (xy -1.767438 -2.807165) (xy -1.81525 -2.840117)
    (xy -1.882495 -2.885273) (xy -1.939436 -2.921057) (xy -1.978646 -2.942938) (xy -1.991381 -2.947563) (xy -2.009917 -2.935085)
    (xy -2.050941 -2.900252) (xy -2.110475 -2.846678) (xy -2.184542 -2.777983) (xy -2.269165 -2.697781) (xy -2.322685 -2.646286)
    (xy -2.416319 -2.554286) (xy -2.497241 -2.471999) (xy -2.562177 -2.402945) (xy -2.607858 -2.350644) (xy -2.631011 -2.318616)
    (xy -2.633232 -2.312116) (xy -2.622924 -2.287394) (xy -2.594439 -2.237405) (xy -2.550937 -2.167212) (xy -2.495577 -2.081875)
    (xy -2.43152 -1.986456) (xy -2.413303 -1.959854) (xy -2.346927 -1.863167) (xy -2.287378 -1.776117) (xy -2.237984 -1.703595)
    (xy -2.202075 -1.650493) (xy -2.182981 -1.621703) (xy -2.181136 -1.618726) (xy -2.183895 -1.595782) (xy -2.198538 -1.545336)
    (xy -2.222513 -1.474041) (xy -2.253266 -1.388547) (xy -2.288244 -1.295507) (xy -2.324893 -1.201574) (xy -2.360661 -1.113399)
    (xy -2.392994 -1.037634) (xy -2.419338 -0.980931) (xy -2.437142 -0.949943) (xy -2.438407 -0.948457) (xy -2.449294 -0.939601)
    (xy -2.467682 -0.930843) (xy -2.497606 -0.921277) (xy -2.543103 -0.909996) (xy -2.608209 -0.896093) (xy -2.696961 -0.878663)
    (xy -2.813393 -0.856798) (xy -2.961542 -0.829591) (xy -2.993618 -0.823741) (xy -3.088686 -0.805374) (xy -3.171565 -0.787405)
    (xy -3.23493 -0.771569) (xy -3.271458 -0.7596) (xy -3.276356 -0.75681) (xy -3.284427 -0.732072) (xy -3.290987 -0.67679)
    (xy -3.296033 -0.597389) (xy -3.299559 -0.500296) (xy -3.301561 -0.391938) (xy -3.302036 -0.27874) (xy -3.300977 -0.167128)
    (xy -3.298382 -0.063529) (xy -3.294246 0.025632) (xy -3.288563 0.093928) (xy -3.281331 0.134934) (xy -3.276971 0.143326)
    (xy -3.252698 0.151792) (xy -3.197426 0.165565) (xy -3.116662 0.18345) (xy -3.015912 0.204252) (xy -2.900683 0.226777)
    (xy -2.837902 0.238582) (xy -2.718787 0.260849) (xy -2.612565 0.281021) (xy -2.524427 0.298085) (xy -2.459566 0.311031)
    (xy -2.423174 0.318845) (xy -2.417184 0.320578) (xy -2.407061 0.34011) (xy -2.385662 0.387157) (xy -2.355839 0.454997)
    (xy -2.320445 0.536909) (xy -2.282332 0.626172) (xy -2.244353 0.716065) (xy -2.20936 0.799865) (xy -2.180206 0.870853)
    (xy -2.159743 0.922306) (xy -2.150823 0.947503) (xy -2.150657 0.948604) (xy -2.160769 0.968481) (xy -2.189117 1.014223)
    (xy -2.232723 1.081283) (xy -2.288606 1.165116) (xy -2.353787 1.261174) (xy -2.391679 1.31635) (xy -2.460725 1.417519)
    (xy -2.52205 1.50937) (xy -2.572663 1.587256) (xy -2.609571 1.646531) (xy -2.629782 1.682549) (xy -2.632701 1.690623)
    (xy -2.620153 1.709416) (xy -2.585463 1.749543) (xy -2.533063 1.806507) (xy -2.467384 1.875815) (xy -2.392856 1.952969)
    (xy -2.313913 2.033475) (xy -2.234983 2.112837) (xy -2.1605 2.18656) (xy -2.094894 2.250148) (xy -2.042596 2.299106)
    (xy -2.008039 2.328939) (xy -1.996478 2.336058) (xy -1.977654 2.326047) (xy -1.932631 2.297922) (xy -1.865787 2.254546)
    (xy -1.781499 2.198782) (xy -1.684144 2.133494) (xy -1.610707 2.083754) (xy -1.239667 1.831449) (xy -0.621095 2.086445)
    (xy -0.537275 2.531069) (xy -0.453454 2.975693) (xy 0.471994 2.975693) (xy 0.555814 2.531069))
   (layer B.Cu) (width 0.01)))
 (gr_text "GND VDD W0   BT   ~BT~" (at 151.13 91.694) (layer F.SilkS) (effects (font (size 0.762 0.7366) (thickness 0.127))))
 (gr_line (start 137.16 96.52) (end 137.16 78.74) (layer Edge.Cuts) (width 0.0254))
 (gr_line (start 165.1 96.52) (end 137.16 96.52) (layer Edge.Cuts) (width 0.0254))
 (gr_line (start 165.1 78.74) (end 165.1 96.52) (layer Edge.Cuts) (width 0.0254))
 (gr_line (start 137.16 78.74) (end 165.1 78.74) (layer Edge.Cuts) (width 0.0254))
 (segment (start 138.92 85.41) (end 139.47 85.41) (width 0.25) (layer F.Cu) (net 3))
 (segment (start 138.194999 86.135001) (end 138.92 85.41) (width 0.25) (layer F.Cu) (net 3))
 (segment (start 138.194999 88.410001) (end 138.194999 86.135001) (width 0.25) (layer F.Cu) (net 3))
 (segment (start 144.939999 95.155001) (end 138.194999 88.410001) (width 0.25) (layer F.Cu) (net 3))
 (segment (start 149.954999 95.155001) (end 144.939999 95.155001) (width 0.25) (layer F.Cu) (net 3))
 (segment (start 151.13 93.98) (end 149.954999 95.155001) (width 0.25) (layer F.Cu) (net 3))
 (segment (start 160.99 85.41) (end 159.79 85.41) (width 0.25) (layer F.Cu) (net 3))
 (segment (start 163.775002 85.41) (end 160.99 85.41) (width 0.25) (layer F.Cu) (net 3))
 (segment (start 164.065001 87.864001) (end 164.065001 85.699999) (width 0.25) (layer F.Cu) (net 3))
 (segment (start 164.065001 85.699999) (end 163.775002 85.41) (width 0.25) (layer F.Cu) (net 3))
 (segment (start 156.774001 95.155001) (end 164.065001 87.864001) (width 0.25) (layer F.Cu) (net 3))
 (segment (start 152.305001 95.155001) (end 156.774001 95.155001) (width 0.25) (layer F.Cu) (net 3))
 (segment (start 151.13 93.98) (end 152.305001 95.155001) (width 0.25) (layer F.Cu) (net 3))
 (segment (start 154.29 81.05) (end 153.504 80.264) (width 0.25) (layer F.Cu) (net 2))
 (segment (start 146.37 81.05) (end 146.37 80.5) (width 0.25) (layer F.Cu) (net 2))
 (segment (start 151.13 91.44) (end 151.13 80.829685) (width 0.25) (layer B.Cu) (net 2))
 (segment (start 151.13 80.829685) (end 151.13 80.264) (width 0.25) (layer B.Cu) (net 2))
 (segment (start 150.622 79.756) (end 150.730001 79.864001) (width 0.25) (layer F.Cu) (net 2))
 (segment (start 151.695685 80.264) (end 151.13 80.264) (width 0.25) (layer F.Cu) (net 2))
 (segment (start 153.504 80.264) (end 151.695685 80.264) (width 0.25) (layer F.Cu) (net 2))
 (segment (start 148.59 93.98) (end 151.13 91.44) (width 0.25) (layer B.Cu) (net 2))
 (segment (start 146.37 80.5) (end 147.114 79.756) (width 0.25) (layer F.Cu) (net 2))
 (segment (start 154.94 81.05) (end 154.29 81.05) (width 0.25) (layer F.Cu) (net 2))
 (segment (start 147.114 79.756) (end 150.622 79.756) (width 0.25) (layer F.Cu) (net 2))
 (segment (start 150.730001 79.864001) (end 151.13 80.264) (width 0.25) (layer F.Cu) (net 2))
 (via (at 151.13 80.264) (size 0.8) (drill 0.4) (layers F.Cu B.Cu) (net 2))
 (segment (start 147.97 90.4) (end 147.32 90.4) (width 0.25) (layer F.Cu) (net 1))
 (segment (start 148.42001 90.85001) (end 147.97 90.4) (width 0.25) (layer F.Cu) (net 1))
 (segment (start 151.17642 90.85001) (end 148.42001 90.85001) (width 0.25) (layer F.Cu) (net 1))
 (segment (start 152.001411 91.675001) (end 151.17642 90.85001) (width 0.25) (layer F.Cu) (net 1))
 (segment (start 155.164999 91.675001) (end 152.001411 91.675001) (width 0.25) (layer F.Cu) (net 1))
 (segment (start 155.89 90.95) (end 155.164999 91.675001) (width 0.25) (layer F.Cu) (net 1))
 (segment (start 155.89 90.4) (end 155.89 90.95) (width 0.25) (layer F.Cu) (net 1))
 (via (at 146.05 90.424) (size 0.8) (drill 0.4) (layers F.Cu B.Cu) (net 1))
 (segment (start 146.074 90.4) (end 146.05 90.424) (width 0.25) (layer F.Cu) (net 1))
 (segment (start 147.32 90.4) (end 146.074 90.4) (width 0.25) (layer F.Cu) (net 1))
 (segment (start 146.05 90.424) (end 146.05 93.98) (width 0.25) (layer B.Cu) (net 1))
 (segment (start 153.99 84.05) (end 153.99 90.4) (width 0.25) (layer F.Cu) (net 6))
 (segment (start 146.67 84.05) (end 147.32 84.05) (width 0.25) (layer F.Cu) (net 6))
 (segment (start 146.37 84.35) (end 146.67 84.05) (width 0.25) (layer F.Cu) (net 6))
 (segment (start 146.37 87.4) (end 146.37 84.35) (width 0.25) (layer F.Cu) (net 6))
 (segment (start 145.72 87.4) (end 146.37 87.4) (width 0.25) (layer F.Cu) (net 6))
 (segment (start 142.86 87.4) (end 145.72 87.4) (width 0.25) (layer F.Cu) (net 6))
 (segment (start 142.47 87.01) (end 142.86 87.4) (width 0.25) (layer F.Cu) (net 6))
 (segment (start 142.47 86.36) (end 142.47 87.01) (width 0.25) (layer F.Cu) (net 6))
 (segment (start 146.37 87.95) (end 146.37 87.4) (width 0.25) (layer F.Cu) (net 6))
 (segment (start 147.02 88.6) (end 146.37 87.95) (width 0.25) (layer F.Cu) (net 6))
 (segment (start 147.57 88.6) (end 147.02 88.6) (width 0.25) (layer F.Cu) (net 6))
 (segment (start 149.37 90.4) (end 147.57 88.6) (width 0.25) (layer F.Cu) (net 6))
 (segment (start 153.99 90.4) (end 149.37 90.4) (width 0.25) (layer F.Cu) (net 6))
 (segment (start 148.27 82.25) (end 148.27 87.4) (width 0.25) (layer F.Cu) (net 7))
 (segment (start 148.27 81.05) (end 148.27 82.25) (width 0.25) (layer F.Cu) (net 7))
 (segment (start 154.94 84.35) (end 155.24 84.05) (width 0.25) (layer F.Cu) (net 7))
 (segment (start 155.24 84.05) (end 155.89 84.05) (width 0.25) (layer F.Cu) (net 7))
 (segment (start 154.94 87.4) (end 154.94 84.35) (width 0.25) (layer F.Cu) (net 7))
 (segment (start 155.03 87.31) (end 154.94 87.4) (width 0.25) (layer F.Cu) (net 7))
 (segment (start 159.79 87.31) (end 155.03 87.31) (width 0.25) (layer F.Cu) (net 7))
 (segment (start 155.24 82.85) (end 155.89 83.5) (width 0.25) (layer F.Cu) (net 7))
 (segment (start 154.69 82.85) (end 155.24 82.85) (width 0.25) (layer F.Cu) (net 7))
 (segment (start 155.89 83.5) (end 155.89 84.05) (width 0.25) (layer F.Cu) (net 7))
 (segment (start 148.27 81.05) (end 152.89 81.05) (width 0.25) (layer F.Cu) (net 7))
 (segment (start 152.89 81.05) (end 154.69 82.85) (width 0.25) (layer F.Cu) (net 7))
 (segment (start 145.035001 91.675001) (end 140.67 87.31) (width 0.25) (layer F.Cu) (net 4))
 (segment (start 151.365001 91.675001) (end 145.035001 91.675001) (width 0.25) (layer F.Cu) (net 4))
 (segment (start 140.67 87.31) (end 139.47 87.31) (width 0.25) (layer F.Cu) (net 4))
 (segment (start 153.67 93.98) (end 151.365001 91.675001) (width 0.25) (layer F.Cu) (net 4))
 (segment (start 162.79 87.4) (end 162.79 86.36) (width 0.25) (layer F.Cu) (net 5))
 (segment (start 156.21 93.98) (end 162.79 87.4) (width 0.25) (layer F.Cu) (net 5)))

